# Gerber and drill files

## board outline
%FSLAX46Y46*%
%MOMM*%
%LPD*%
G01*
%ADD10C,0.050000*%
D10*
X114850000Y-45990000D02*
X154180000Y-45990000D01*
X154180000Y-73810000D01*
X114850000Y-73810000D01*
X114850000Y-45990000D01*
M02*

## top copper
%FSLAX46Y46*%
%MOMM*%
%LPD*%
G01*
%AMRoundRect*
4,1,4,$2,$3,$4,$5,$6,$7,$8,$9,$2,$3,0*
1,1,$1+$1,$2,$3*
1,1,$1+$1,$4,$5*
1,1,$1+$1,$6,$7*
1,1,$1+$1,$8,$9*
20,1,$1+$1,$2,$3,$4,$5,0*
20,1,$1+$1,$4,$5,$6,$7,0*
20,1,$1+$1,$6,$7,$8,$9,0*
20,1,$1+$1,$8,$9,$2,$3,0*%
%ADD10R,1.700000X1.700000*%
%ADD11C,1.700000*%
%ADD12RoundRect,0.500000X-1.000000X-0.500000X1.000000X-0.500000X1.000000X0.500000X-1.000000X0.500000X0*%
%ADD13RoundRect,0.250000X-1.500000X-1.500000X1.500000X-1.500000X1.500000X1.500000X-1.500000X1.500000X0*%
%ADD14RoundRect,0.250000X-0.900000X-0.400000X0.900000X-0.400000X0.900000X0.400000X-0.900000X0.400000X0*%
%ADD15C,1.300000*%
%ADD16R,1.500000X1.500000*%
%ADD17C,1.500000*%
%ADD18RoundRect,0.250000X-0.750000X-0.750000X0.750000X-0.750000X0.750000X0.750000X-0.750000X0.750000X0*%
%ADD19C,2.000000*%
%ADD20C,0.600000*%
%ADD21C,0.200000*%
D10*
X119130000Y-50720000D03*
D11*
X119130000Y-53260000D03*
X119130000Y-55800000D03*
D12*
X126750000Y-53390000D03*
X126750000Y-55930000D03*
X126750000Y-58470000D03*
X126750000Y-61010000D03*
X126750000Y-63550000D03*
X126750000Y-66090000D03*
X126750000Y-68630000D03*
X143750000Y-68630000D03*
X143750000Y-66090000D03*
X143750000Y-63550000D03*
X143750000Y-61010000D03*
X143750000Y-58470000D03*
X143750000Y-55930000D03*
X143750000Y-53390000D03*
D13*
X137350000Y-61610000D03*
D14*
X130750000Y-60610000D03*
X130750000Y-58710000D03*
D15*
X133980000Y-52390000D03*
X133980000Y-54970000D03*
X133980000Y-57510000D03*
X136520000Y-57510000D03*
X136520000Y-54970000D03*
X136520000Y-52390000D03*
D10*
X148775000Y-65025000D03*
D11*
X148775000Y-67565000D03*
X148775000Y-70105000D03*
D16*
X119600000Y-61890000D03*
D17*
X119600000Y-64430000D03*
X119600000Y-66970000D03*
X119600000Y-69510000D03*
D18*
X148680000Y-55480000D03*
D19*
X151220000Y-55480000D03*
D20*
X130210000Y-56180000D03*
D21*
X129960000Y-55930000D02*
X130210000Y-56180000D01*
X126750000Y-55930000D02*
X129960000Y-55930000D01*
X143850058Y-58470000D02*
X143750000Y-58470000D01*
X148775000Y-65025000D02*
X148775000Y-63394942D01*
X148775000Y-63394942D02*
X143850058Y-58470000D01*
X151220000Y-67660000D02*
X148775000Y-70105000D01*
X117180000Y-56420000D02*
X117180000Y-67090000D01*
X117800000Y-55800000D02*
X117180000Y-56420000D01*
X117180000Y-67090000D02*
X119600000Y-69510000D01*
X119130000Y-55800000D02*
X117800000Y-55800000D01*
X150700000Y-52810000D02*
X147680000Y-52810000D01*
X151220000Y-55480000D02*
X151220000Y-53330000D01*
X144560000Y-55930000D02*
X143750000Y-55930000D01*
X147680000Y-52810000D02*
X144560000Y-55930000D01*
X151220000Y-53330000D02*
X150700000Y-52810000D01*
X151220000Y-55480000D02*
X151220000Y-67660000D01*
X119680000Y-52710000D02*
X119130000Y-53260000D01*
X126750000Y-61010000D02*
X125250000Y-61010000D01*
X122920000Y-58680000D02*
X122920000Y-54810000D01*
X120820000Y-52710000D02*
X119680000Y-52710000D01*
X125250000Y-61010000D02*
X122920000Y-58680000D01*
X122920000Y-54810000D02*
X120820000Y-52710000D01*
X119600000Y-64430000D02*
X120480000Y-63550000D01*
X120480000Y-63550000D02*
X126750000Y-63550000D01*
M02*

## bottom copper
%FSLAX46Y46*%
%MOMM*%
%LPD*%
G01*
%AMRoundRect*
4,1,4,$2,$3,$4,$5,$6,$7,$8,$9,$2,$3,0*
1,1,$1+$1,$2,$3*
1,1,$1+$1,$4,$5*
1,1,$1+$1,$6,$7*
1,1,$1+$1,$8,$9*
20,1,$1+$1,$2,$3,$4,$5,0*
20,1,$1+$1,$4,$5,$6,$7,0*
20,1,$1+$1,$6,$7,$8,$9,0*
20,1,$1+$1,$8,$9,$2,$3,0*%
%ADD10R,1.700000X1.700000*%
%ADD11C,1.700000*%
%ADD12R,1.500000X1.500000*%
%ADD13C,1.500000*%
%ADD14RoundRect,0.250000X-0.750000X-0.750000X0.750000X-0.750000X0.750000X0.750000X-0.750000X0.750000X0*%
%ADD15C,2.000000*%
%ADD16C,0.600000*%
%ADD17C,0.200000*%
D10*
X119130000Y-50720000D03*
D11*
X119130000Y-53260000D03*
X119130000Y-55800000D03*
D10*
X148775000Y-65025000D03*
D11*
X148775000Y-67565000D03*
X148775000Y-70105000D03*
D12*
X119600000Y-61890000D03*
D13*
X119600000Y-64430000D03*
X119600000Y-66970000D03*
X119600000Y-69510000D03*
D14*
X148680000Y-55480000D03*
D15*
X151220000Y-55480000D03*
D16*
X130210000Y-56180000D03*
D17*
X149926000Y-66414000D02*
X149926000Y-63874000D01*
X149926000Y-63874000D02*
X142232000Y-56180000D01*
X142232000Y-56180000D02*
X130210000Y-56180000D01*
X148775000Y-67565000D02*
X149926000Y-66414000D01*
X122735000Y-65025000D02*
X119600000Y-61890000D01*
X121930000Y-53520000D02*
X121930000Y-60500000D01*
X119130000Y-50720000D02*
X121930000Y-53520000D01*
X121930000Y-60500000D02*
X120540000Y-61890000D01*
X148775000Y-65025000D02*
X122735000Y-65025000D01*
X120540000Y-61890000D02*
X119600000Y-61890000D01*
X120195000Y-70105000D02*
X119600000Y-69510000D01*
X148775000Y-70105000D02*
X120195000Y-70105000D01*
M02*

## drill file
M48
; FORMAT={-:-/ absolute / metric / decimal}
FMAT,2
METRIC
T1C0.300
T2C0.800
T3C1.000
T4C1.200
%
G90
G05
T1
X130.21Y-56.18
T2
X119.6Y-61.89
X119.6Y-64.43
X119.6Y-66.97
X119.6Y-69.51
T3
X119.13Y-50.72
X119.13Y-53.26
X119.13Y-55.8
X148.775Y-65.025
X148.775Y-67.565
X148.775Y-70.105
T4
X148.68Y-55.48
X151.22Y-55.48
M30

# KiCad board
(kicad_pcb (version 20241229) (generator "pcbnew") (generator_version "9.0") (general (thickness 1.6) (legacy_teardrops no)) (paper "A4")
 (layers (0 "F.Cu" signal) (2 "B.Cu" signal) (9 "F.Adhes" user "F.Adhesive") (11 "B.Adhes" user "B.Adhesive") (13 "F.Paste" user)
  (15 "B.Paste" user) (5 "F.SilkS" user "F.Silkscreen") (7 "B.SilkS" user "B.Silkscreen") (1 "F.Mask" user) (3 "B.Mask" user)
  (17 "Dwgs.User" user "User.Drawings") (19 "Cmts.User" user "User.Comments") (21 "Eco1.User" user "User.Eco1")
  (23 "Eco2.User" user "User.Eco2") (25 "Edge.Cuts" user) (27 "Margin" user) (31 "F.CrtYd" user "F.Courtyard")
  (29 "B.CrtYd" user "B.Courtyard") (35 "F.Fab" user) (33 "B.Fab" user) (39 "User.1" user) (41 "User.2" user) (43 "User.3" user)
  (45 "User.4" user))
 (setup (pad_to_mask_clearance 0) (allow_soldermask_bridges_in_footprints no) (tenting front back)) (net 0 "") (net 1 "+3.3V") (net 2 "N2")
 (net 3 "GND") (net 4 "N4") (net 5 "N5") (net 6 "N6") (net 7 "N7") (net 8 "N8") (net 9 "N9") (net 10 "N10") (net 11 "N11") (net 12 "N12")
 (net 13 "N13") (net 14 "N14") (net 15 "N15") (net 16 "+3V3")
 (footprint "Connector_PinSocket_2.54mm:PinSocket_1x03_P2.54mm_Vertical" (layer "F.Cu") (at 119.13 50.72)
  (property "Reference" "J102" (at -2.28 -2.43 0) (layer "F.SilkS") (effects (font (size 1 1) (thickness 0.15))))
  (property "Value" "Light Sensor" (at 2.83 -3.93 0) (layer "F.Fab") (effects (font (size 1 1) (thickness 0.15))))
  (pad "1" thru_hole rect (at 0 0) (size 1.7 1.7) (drill 1) (layers "*.Cu" "*.Mask") (remove_unused_layers no) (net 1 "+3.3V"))
  (pad "2" thru_hole circle (at 0 2.54) (size 1.7 1.7) (drill 1) (layers "*.Cu" "*.Mask") (remove_unused_layers no) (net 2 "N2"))
  (pad "3" thru_hole circle (at 0 5.08) (size 1.7 1.7) (drill 1) (layers "*.Cu" "*.Mask") (remove_unused_layers no) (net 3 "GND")))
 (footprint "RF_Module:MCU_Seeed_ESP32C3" (layer "F.Cu") (at 135.25 61.01)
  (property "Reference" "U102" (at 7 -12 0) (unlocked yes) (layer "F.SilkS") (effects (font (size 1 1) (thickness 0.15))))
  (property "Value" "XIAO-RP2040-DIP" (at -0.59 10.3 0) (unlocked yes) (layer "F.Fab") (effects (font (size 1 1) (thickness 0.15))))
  (pad "" smd roundrect (at 1.1 -0.4) (size 1.5 1.5) (layers "F.Paste") (roundrect_rratio 0.1666666667))
  (pad "" smd roundrect (at 1.1 1.6) (size 1.5 1.5) (layers "F.Paste") (roundrect_rratio 0.1666666667))
  (pad "" smd roundrect (at 3.1 -0.4) (size 1.5 1.5) (layers "F.Paste") (roundrect_rratio 0.1666666667))
  (pad "" smd roundrect (at 3.1 1.6) (size 1.5 1.5) (layers "F.Paste") (roundrect_rratio 0.1666666667))
  (pad "1" smd roundrect (at -8.5 -7.62) (size 3 2) (layers "F.Cu" "F.Mask" "F.Paste") (roundrect_rratio 0.25) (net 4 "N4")
   (thermal_bridge_angle 45))
  (pad "2" smd roundrect (at -8.5 -5.08) (size 3 2) (layers "F.Cu" "F.Mask" "F.Paste") (roundrect_rratio 0.25) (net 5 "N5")
   (thermal_bridge_angle 45))
  (pad "3" smd roundrect (at -8.5 -2.54) (size 3 2) (layers "F.Cu" "F.Mask" "F.Paste") (roundrect_rratio 0.25) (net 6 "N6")
   (thermal_bridge_angle 45))
  (pad "4" smd roundrect (at -8.5 0) (size 3 2) (layers "F.Cu" "F.Mask" "F.Paste") (roundrect_rratio 0.25) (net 2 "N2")
   (thermal_bridge_angle 45))
  (pad "5" smd roundrect (at -8.5 2.54) (size 3 2) (layers "F.Cu" "F.Mask" "F.Paste") (roundrect_rratio 0.25) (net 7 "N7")
   (thermal_bridge_angle 45))
  (pad "6" smd roundrect (at -8.5 5.08) (size 3 2) (layers "F.Cu" "F.Mask" "F.Paste") (roundrect_rratio 0.25) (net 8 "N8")
   (thermal_bridge_angle 45))
  (pad "7" smd roundrect (at -8.5 7.62) (size 3 2) (layers "F.Cu" "F.Mask" "F.Paste") (roundrect_rratio 0.25) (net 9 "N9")
   (thermal_bridge_angle 45))
  (pad "8" smd roundrect (at 8.5 7.62) (size 3 2) (layers "F.Cu" "F.Mask" "F.Paste") (roundrect_rratio 0.25) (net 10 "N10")
   (thermal_bridge_angle 45))
  (pad "9" smd roundrect (at 8.5 5.08) (size 3 2) (layers "F.Cu" "F.Mask" "F.Paste") (roundrect_rratio 0.25) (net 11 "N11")
   (thermal_bridge_angle 45))
  (pad "10" smd roundrect (at 8.5 2.54) (size 3 2) (layers "F.Cu" "F.Mask" "F.Paste") (roundrect_rratio 0.25) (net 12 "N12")
   (thermal_bridge_angle 45))
  (pad "11" smd roundrect (at 8.5 0) (size 3 2) (layers "F.Cu" "F.Mask" "F.Paste") (roundrect_rratio 0.25) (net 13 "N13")
   (thermal_bridge_angle 45))
  (pad "12" smd roundrect (at 8.5 -2.54) (size 3 2) (layers "F.Cu" "F.Mask" "F.Paste") (roundrect_rratio 0.25) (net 1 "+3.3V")
   (thermal_bridge_angle 45))
  (pad "13" smd roundrect (at 8.5 -5.08) (size 3 2) (layers "F.Cu" "F.Mask" "F.Paste") (roundrect_rratio 0.25) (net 3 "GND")
   (thermal_bridge_angle 45))
  (pad "14" smd roundrect (at 8.5 -7.62) (size 3 2) (layers "F.Cu" "F.Mask" "F.Paste") (roundrect_rratio 0.25) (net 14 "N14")
   (thermal_bridge_angle 45))
  (pad "15" smd roundrect (at 2.1 0.6) (size 3.5 3.5) (layers "F.Cu" "F.Mask") (roundrect_rratio 0.07142857143))
  (pad "16" smd roundrect (at -4.5 -0.4) (size 2.3 1.3) (layers "F.Cu" "F.Mask" "F.Paste") (roundrect_rratio 0.1923076923))
  (pad "17" smd roundrect (at -4.5 -2.3) (size 2.3 1.3) (layers "F.Cu" "F.Mask" "F.Paste") (roundrect_rratio 0.1923076923))
  (pad "18" smd circle (at -1.27 -8.62) (size 1.3 1.3) (layers "F.Cu" "F.Mask" "F.Paste"))
  (pad "19" smd circle (at -1.27 -6.04) (size 1.3 1.3) (layers "F.Cu" "F.Mask" "F.Paste"))
  (pad "20" smd circle (at -1.27 -3.5) (size 1.3 1.3) (layers "F.Cu" "F.Mask" "F.Paste"))
  (pad "21" smd circle (at 1.27 -3.5) (size 1.3 1.3) (layers "F.Cu" "F.Mask" "F.Paste"))
  (pad "22" smd circle (at 1.27 -6.04) (size 1.3 1.3) (layers "F.Cu" "F.Mask" "F.Paste"))
  (pad "23" smd circle (at 1.27 -8.62) (size 1.3 1.3) (layers "F.Cu" "F.Mask" "F.Paste")))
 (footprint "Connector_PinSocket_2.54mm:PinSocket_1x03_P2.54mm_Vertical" (layer "F.Cu") (at 148.775 65.025)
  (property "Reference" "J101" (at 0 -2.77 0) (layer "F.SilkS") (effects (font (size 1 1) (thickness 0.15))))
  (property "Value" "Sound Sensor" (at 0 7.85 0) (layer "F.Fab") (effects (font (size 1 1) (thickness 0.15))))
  (pad "1" thru_hole rect (at 0 0) (size 1.7 1.7) (drill 1) (layers "*.Cu" "*.Mask") (remove_unused_layers no) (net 1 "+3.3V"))
  (pad "2" thru_hole circle (at 0 2.54) (size 1.7 1.7) (drill 1) (layers "*.Cu" "*.Mask") (remove_unused_layers no) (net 5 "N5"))
  (pad "3" thru_hole circle (at 0 5.08) (size 1.7 1.7) (drill 1) (layers "*.Cu" "*.Mask") (remove_unused_layers no) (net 3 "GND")))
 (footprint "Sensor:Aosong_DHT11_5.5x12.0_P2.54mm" (layer "F.Cu") (at 119.6 61.89)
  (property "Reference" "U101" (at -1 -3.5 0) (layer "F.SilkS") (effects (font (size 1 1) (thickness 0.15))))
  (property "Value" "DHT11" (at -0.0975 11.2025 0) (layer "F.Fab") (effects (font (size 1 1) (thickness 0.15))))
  (pad "1" thru_hole rect (at 0 0) (size 1.5 1.5) (drill 0.8) (layers "*.Cu" "*.Mask") (remove_unused_layers no) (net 1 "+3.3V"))
  (pad "2" thru_hole circle (at 0 2.54) (size 1.5 1.5) (drill 0.8) (layers "*.Cu" "*.Mask") (remove_unused_layers no) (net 7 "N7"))
  (pad "3" thru_hole circle (at 0 5.08) (size 1.5 1.5) (drill 0.8) (layers "*.Cu" "*.Mask") (remove_unused_layers no) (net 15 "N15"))
  (pad "4" thru_hole circle (at 0 7.62) (size 1.5 1.5) (drill 0.8) (layers "*.Cu" "*.Mask") (remove_unused_layers no) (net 3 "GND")))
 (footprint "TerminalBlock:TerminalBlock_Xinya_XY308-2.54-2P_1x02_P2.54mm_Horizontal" (layer "F.Cu") (at 148.68 55.48)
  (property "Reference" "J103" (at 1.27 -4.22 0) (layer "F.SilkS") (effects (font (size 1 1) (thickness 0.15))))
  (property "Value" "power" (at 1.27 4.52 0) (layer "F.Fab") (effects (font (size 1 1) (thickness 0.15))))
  (pad "1" thru_hole roundrect (at 0 0) (size 2 2) (drill 1.2) (layers "*.Cu" "*.Mask") (remove_unused_layers no) (roundrect_rratio 0.125)
   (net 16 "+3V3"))
  (pad "2" thru_hole circle (at 2.54 0) (size 2 2) (drill 1.2) (layers "*.Cu" "*.Mask") (remove_unused_layers no) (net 3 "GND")))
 (gr_rect (start 114.85 45.99) (end 154.18 73.81) (stroke (width 0.05) (type default)) (fill no) (layer "Edge.Cuts"))
 (segment (start 129.96 55.93) (end 130.21 56.18) (width 0.2) (layer "F.Cu") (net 5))
 (segment (start 126.75 55.93) (end 129.96 55.93) (width 0.2) (layer "F.Cu") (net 5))
 (via (at 130.21 56.18) (size 0.6) (drill 0.3) (layers "F.Cu" "B.Cu") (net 5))
 (segment (start 149.926 66.414) (end 149.926 63.874) (width 0.2) (layer "B.Cu") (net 5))
 (segment (start 149.926 63.874) (end 142.232 56.18) (width 0.2) (layer "B.Cu") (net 5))
 (segment (start 142.232 56.18) (end 130.21 56.18) (width 0.2) (layer "B.Cu") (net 5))
 (segment (start 148.775 67.565) (end 149.926 66.414) (width 0.2) (layer "B.Cu") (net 5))
 (segment (start 143.850058 58.47) (end 143.75 58.47) (width 0.2) (layer "F.Cu") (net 1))
 (segment (start 148.775 65.025) (end 148.775 63.394942) (width 0.2) (layer "F.Cu") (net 1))
 (segment (start 148.775 63.394942) (end 143.850058 58.47) (width 0.2) (layer "F.Cu") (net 1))
 (segment (start 122.735 65.025) (end 119.6 61.89) (width 0.2) (layer "B.Cu") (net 1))
 (segment (start 121.93 53.52) (end 121.93 60.5) (width 0.2) (layer "B.Cu") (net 1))
 (segment (start 119.13 50.72) (end 121.93 53.52) (width 0.2) (layer "B.Cu") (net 1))
 (segment (start 121.93 60.5) (end 120.54 61.89) (width 0.2) (layer "B.Cu") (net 1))
 (segment (start 148.775 65.025) (end 122.735 65.025) (width 0.2) (layer "B.Cu") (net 1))
 (segment (start 120.54 61.89) (end 119.6 61.89) (width 0.2) (layer "B.Cu") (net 1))
 (segment (start 151.22 67.66) (end 148.775 70.105) (width 0.2) (layer "F.Cu") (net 3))
 (segment (start 117.18 56.42) (end 117.18 67.09) (width 0.2) (layer "F.Cu") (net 3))
 (segment (start 117.8 55.8) (end 117.18 56.42) (width 0.2) (layer "F.Cu") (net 3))
 (segment (start 117.18 67.09) (end 119.6 69.51) (width 0.2) (layer "F.Cu") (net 3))
 (segment (start 119.13 55.8) (end 117.8 55.8) (width 0.2) (layer "F.Cu") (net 3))
 (segment (start 150.7 52.81) (end 147.68 52.81) (width 0.2) (layer "F.Cu") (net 3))
 (segment (start 151.22 55.48) (end 151.22 53.33) (width 0.2) (layer "F.Cu") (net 3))
 (segment (start 144.56 55.93) (end 143.75 55.93) (width 0.2) (layer "F.Cu") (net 3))
 (segment (start 147.68 52.81) (end 144.56 55.93) (width 0.2) (layer "F.Cu") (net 3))
 (segment (start 151.22 53.33) (end 150.7 52.81) (width 0.2) (layer "F.Cu") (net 3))
 (segment (start 151.22 55.48) (end 151.22 67.66) (width 0.2) (layer "F.Cu") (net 3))
 (segment (start 120.195 70.105) (end 119.6 69.51) (width 0.2) (layer "B.Cu") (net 3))
 (segment (start 148.775 70.105) (end 120.195 70.105) (width 0.2) (layer "B.Cu") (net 3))
 (segment (start 119.68 52.71) (end 119.13 53.26) (width 0.2) (layer "F.Cu") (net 2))
 (segment (start 126.75 61.01) (end 125.25 61.01) (width 0.2) (layer "F.Cu") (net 2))
 (segment (start 122.92 58.68) (end 122.92 54.81) (width 0.2) (layer "F.Cu") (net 2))
 (segment (start 120.82 52.71) (end 119.68 52.71) (width 0.2) (layer "F.Cu") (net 2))
 (segment (start 125.25 61.01) (end 122.92 58.68) (width 0.2) (layer "F.Cu") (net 2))
 (segment (start 122.92 54.81) (end 120.82 52.71) (width 0.2) (layer "F.Cu") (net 2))
 (segment (start 119.6 64.43) (end 120.48 63.55) (width 0.2) (layer "F.Cu") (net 7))
 (segment (start 120.48 63.55) (end 126.75 63.55) (width 0.2) (layer "F.Cu") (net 7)))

